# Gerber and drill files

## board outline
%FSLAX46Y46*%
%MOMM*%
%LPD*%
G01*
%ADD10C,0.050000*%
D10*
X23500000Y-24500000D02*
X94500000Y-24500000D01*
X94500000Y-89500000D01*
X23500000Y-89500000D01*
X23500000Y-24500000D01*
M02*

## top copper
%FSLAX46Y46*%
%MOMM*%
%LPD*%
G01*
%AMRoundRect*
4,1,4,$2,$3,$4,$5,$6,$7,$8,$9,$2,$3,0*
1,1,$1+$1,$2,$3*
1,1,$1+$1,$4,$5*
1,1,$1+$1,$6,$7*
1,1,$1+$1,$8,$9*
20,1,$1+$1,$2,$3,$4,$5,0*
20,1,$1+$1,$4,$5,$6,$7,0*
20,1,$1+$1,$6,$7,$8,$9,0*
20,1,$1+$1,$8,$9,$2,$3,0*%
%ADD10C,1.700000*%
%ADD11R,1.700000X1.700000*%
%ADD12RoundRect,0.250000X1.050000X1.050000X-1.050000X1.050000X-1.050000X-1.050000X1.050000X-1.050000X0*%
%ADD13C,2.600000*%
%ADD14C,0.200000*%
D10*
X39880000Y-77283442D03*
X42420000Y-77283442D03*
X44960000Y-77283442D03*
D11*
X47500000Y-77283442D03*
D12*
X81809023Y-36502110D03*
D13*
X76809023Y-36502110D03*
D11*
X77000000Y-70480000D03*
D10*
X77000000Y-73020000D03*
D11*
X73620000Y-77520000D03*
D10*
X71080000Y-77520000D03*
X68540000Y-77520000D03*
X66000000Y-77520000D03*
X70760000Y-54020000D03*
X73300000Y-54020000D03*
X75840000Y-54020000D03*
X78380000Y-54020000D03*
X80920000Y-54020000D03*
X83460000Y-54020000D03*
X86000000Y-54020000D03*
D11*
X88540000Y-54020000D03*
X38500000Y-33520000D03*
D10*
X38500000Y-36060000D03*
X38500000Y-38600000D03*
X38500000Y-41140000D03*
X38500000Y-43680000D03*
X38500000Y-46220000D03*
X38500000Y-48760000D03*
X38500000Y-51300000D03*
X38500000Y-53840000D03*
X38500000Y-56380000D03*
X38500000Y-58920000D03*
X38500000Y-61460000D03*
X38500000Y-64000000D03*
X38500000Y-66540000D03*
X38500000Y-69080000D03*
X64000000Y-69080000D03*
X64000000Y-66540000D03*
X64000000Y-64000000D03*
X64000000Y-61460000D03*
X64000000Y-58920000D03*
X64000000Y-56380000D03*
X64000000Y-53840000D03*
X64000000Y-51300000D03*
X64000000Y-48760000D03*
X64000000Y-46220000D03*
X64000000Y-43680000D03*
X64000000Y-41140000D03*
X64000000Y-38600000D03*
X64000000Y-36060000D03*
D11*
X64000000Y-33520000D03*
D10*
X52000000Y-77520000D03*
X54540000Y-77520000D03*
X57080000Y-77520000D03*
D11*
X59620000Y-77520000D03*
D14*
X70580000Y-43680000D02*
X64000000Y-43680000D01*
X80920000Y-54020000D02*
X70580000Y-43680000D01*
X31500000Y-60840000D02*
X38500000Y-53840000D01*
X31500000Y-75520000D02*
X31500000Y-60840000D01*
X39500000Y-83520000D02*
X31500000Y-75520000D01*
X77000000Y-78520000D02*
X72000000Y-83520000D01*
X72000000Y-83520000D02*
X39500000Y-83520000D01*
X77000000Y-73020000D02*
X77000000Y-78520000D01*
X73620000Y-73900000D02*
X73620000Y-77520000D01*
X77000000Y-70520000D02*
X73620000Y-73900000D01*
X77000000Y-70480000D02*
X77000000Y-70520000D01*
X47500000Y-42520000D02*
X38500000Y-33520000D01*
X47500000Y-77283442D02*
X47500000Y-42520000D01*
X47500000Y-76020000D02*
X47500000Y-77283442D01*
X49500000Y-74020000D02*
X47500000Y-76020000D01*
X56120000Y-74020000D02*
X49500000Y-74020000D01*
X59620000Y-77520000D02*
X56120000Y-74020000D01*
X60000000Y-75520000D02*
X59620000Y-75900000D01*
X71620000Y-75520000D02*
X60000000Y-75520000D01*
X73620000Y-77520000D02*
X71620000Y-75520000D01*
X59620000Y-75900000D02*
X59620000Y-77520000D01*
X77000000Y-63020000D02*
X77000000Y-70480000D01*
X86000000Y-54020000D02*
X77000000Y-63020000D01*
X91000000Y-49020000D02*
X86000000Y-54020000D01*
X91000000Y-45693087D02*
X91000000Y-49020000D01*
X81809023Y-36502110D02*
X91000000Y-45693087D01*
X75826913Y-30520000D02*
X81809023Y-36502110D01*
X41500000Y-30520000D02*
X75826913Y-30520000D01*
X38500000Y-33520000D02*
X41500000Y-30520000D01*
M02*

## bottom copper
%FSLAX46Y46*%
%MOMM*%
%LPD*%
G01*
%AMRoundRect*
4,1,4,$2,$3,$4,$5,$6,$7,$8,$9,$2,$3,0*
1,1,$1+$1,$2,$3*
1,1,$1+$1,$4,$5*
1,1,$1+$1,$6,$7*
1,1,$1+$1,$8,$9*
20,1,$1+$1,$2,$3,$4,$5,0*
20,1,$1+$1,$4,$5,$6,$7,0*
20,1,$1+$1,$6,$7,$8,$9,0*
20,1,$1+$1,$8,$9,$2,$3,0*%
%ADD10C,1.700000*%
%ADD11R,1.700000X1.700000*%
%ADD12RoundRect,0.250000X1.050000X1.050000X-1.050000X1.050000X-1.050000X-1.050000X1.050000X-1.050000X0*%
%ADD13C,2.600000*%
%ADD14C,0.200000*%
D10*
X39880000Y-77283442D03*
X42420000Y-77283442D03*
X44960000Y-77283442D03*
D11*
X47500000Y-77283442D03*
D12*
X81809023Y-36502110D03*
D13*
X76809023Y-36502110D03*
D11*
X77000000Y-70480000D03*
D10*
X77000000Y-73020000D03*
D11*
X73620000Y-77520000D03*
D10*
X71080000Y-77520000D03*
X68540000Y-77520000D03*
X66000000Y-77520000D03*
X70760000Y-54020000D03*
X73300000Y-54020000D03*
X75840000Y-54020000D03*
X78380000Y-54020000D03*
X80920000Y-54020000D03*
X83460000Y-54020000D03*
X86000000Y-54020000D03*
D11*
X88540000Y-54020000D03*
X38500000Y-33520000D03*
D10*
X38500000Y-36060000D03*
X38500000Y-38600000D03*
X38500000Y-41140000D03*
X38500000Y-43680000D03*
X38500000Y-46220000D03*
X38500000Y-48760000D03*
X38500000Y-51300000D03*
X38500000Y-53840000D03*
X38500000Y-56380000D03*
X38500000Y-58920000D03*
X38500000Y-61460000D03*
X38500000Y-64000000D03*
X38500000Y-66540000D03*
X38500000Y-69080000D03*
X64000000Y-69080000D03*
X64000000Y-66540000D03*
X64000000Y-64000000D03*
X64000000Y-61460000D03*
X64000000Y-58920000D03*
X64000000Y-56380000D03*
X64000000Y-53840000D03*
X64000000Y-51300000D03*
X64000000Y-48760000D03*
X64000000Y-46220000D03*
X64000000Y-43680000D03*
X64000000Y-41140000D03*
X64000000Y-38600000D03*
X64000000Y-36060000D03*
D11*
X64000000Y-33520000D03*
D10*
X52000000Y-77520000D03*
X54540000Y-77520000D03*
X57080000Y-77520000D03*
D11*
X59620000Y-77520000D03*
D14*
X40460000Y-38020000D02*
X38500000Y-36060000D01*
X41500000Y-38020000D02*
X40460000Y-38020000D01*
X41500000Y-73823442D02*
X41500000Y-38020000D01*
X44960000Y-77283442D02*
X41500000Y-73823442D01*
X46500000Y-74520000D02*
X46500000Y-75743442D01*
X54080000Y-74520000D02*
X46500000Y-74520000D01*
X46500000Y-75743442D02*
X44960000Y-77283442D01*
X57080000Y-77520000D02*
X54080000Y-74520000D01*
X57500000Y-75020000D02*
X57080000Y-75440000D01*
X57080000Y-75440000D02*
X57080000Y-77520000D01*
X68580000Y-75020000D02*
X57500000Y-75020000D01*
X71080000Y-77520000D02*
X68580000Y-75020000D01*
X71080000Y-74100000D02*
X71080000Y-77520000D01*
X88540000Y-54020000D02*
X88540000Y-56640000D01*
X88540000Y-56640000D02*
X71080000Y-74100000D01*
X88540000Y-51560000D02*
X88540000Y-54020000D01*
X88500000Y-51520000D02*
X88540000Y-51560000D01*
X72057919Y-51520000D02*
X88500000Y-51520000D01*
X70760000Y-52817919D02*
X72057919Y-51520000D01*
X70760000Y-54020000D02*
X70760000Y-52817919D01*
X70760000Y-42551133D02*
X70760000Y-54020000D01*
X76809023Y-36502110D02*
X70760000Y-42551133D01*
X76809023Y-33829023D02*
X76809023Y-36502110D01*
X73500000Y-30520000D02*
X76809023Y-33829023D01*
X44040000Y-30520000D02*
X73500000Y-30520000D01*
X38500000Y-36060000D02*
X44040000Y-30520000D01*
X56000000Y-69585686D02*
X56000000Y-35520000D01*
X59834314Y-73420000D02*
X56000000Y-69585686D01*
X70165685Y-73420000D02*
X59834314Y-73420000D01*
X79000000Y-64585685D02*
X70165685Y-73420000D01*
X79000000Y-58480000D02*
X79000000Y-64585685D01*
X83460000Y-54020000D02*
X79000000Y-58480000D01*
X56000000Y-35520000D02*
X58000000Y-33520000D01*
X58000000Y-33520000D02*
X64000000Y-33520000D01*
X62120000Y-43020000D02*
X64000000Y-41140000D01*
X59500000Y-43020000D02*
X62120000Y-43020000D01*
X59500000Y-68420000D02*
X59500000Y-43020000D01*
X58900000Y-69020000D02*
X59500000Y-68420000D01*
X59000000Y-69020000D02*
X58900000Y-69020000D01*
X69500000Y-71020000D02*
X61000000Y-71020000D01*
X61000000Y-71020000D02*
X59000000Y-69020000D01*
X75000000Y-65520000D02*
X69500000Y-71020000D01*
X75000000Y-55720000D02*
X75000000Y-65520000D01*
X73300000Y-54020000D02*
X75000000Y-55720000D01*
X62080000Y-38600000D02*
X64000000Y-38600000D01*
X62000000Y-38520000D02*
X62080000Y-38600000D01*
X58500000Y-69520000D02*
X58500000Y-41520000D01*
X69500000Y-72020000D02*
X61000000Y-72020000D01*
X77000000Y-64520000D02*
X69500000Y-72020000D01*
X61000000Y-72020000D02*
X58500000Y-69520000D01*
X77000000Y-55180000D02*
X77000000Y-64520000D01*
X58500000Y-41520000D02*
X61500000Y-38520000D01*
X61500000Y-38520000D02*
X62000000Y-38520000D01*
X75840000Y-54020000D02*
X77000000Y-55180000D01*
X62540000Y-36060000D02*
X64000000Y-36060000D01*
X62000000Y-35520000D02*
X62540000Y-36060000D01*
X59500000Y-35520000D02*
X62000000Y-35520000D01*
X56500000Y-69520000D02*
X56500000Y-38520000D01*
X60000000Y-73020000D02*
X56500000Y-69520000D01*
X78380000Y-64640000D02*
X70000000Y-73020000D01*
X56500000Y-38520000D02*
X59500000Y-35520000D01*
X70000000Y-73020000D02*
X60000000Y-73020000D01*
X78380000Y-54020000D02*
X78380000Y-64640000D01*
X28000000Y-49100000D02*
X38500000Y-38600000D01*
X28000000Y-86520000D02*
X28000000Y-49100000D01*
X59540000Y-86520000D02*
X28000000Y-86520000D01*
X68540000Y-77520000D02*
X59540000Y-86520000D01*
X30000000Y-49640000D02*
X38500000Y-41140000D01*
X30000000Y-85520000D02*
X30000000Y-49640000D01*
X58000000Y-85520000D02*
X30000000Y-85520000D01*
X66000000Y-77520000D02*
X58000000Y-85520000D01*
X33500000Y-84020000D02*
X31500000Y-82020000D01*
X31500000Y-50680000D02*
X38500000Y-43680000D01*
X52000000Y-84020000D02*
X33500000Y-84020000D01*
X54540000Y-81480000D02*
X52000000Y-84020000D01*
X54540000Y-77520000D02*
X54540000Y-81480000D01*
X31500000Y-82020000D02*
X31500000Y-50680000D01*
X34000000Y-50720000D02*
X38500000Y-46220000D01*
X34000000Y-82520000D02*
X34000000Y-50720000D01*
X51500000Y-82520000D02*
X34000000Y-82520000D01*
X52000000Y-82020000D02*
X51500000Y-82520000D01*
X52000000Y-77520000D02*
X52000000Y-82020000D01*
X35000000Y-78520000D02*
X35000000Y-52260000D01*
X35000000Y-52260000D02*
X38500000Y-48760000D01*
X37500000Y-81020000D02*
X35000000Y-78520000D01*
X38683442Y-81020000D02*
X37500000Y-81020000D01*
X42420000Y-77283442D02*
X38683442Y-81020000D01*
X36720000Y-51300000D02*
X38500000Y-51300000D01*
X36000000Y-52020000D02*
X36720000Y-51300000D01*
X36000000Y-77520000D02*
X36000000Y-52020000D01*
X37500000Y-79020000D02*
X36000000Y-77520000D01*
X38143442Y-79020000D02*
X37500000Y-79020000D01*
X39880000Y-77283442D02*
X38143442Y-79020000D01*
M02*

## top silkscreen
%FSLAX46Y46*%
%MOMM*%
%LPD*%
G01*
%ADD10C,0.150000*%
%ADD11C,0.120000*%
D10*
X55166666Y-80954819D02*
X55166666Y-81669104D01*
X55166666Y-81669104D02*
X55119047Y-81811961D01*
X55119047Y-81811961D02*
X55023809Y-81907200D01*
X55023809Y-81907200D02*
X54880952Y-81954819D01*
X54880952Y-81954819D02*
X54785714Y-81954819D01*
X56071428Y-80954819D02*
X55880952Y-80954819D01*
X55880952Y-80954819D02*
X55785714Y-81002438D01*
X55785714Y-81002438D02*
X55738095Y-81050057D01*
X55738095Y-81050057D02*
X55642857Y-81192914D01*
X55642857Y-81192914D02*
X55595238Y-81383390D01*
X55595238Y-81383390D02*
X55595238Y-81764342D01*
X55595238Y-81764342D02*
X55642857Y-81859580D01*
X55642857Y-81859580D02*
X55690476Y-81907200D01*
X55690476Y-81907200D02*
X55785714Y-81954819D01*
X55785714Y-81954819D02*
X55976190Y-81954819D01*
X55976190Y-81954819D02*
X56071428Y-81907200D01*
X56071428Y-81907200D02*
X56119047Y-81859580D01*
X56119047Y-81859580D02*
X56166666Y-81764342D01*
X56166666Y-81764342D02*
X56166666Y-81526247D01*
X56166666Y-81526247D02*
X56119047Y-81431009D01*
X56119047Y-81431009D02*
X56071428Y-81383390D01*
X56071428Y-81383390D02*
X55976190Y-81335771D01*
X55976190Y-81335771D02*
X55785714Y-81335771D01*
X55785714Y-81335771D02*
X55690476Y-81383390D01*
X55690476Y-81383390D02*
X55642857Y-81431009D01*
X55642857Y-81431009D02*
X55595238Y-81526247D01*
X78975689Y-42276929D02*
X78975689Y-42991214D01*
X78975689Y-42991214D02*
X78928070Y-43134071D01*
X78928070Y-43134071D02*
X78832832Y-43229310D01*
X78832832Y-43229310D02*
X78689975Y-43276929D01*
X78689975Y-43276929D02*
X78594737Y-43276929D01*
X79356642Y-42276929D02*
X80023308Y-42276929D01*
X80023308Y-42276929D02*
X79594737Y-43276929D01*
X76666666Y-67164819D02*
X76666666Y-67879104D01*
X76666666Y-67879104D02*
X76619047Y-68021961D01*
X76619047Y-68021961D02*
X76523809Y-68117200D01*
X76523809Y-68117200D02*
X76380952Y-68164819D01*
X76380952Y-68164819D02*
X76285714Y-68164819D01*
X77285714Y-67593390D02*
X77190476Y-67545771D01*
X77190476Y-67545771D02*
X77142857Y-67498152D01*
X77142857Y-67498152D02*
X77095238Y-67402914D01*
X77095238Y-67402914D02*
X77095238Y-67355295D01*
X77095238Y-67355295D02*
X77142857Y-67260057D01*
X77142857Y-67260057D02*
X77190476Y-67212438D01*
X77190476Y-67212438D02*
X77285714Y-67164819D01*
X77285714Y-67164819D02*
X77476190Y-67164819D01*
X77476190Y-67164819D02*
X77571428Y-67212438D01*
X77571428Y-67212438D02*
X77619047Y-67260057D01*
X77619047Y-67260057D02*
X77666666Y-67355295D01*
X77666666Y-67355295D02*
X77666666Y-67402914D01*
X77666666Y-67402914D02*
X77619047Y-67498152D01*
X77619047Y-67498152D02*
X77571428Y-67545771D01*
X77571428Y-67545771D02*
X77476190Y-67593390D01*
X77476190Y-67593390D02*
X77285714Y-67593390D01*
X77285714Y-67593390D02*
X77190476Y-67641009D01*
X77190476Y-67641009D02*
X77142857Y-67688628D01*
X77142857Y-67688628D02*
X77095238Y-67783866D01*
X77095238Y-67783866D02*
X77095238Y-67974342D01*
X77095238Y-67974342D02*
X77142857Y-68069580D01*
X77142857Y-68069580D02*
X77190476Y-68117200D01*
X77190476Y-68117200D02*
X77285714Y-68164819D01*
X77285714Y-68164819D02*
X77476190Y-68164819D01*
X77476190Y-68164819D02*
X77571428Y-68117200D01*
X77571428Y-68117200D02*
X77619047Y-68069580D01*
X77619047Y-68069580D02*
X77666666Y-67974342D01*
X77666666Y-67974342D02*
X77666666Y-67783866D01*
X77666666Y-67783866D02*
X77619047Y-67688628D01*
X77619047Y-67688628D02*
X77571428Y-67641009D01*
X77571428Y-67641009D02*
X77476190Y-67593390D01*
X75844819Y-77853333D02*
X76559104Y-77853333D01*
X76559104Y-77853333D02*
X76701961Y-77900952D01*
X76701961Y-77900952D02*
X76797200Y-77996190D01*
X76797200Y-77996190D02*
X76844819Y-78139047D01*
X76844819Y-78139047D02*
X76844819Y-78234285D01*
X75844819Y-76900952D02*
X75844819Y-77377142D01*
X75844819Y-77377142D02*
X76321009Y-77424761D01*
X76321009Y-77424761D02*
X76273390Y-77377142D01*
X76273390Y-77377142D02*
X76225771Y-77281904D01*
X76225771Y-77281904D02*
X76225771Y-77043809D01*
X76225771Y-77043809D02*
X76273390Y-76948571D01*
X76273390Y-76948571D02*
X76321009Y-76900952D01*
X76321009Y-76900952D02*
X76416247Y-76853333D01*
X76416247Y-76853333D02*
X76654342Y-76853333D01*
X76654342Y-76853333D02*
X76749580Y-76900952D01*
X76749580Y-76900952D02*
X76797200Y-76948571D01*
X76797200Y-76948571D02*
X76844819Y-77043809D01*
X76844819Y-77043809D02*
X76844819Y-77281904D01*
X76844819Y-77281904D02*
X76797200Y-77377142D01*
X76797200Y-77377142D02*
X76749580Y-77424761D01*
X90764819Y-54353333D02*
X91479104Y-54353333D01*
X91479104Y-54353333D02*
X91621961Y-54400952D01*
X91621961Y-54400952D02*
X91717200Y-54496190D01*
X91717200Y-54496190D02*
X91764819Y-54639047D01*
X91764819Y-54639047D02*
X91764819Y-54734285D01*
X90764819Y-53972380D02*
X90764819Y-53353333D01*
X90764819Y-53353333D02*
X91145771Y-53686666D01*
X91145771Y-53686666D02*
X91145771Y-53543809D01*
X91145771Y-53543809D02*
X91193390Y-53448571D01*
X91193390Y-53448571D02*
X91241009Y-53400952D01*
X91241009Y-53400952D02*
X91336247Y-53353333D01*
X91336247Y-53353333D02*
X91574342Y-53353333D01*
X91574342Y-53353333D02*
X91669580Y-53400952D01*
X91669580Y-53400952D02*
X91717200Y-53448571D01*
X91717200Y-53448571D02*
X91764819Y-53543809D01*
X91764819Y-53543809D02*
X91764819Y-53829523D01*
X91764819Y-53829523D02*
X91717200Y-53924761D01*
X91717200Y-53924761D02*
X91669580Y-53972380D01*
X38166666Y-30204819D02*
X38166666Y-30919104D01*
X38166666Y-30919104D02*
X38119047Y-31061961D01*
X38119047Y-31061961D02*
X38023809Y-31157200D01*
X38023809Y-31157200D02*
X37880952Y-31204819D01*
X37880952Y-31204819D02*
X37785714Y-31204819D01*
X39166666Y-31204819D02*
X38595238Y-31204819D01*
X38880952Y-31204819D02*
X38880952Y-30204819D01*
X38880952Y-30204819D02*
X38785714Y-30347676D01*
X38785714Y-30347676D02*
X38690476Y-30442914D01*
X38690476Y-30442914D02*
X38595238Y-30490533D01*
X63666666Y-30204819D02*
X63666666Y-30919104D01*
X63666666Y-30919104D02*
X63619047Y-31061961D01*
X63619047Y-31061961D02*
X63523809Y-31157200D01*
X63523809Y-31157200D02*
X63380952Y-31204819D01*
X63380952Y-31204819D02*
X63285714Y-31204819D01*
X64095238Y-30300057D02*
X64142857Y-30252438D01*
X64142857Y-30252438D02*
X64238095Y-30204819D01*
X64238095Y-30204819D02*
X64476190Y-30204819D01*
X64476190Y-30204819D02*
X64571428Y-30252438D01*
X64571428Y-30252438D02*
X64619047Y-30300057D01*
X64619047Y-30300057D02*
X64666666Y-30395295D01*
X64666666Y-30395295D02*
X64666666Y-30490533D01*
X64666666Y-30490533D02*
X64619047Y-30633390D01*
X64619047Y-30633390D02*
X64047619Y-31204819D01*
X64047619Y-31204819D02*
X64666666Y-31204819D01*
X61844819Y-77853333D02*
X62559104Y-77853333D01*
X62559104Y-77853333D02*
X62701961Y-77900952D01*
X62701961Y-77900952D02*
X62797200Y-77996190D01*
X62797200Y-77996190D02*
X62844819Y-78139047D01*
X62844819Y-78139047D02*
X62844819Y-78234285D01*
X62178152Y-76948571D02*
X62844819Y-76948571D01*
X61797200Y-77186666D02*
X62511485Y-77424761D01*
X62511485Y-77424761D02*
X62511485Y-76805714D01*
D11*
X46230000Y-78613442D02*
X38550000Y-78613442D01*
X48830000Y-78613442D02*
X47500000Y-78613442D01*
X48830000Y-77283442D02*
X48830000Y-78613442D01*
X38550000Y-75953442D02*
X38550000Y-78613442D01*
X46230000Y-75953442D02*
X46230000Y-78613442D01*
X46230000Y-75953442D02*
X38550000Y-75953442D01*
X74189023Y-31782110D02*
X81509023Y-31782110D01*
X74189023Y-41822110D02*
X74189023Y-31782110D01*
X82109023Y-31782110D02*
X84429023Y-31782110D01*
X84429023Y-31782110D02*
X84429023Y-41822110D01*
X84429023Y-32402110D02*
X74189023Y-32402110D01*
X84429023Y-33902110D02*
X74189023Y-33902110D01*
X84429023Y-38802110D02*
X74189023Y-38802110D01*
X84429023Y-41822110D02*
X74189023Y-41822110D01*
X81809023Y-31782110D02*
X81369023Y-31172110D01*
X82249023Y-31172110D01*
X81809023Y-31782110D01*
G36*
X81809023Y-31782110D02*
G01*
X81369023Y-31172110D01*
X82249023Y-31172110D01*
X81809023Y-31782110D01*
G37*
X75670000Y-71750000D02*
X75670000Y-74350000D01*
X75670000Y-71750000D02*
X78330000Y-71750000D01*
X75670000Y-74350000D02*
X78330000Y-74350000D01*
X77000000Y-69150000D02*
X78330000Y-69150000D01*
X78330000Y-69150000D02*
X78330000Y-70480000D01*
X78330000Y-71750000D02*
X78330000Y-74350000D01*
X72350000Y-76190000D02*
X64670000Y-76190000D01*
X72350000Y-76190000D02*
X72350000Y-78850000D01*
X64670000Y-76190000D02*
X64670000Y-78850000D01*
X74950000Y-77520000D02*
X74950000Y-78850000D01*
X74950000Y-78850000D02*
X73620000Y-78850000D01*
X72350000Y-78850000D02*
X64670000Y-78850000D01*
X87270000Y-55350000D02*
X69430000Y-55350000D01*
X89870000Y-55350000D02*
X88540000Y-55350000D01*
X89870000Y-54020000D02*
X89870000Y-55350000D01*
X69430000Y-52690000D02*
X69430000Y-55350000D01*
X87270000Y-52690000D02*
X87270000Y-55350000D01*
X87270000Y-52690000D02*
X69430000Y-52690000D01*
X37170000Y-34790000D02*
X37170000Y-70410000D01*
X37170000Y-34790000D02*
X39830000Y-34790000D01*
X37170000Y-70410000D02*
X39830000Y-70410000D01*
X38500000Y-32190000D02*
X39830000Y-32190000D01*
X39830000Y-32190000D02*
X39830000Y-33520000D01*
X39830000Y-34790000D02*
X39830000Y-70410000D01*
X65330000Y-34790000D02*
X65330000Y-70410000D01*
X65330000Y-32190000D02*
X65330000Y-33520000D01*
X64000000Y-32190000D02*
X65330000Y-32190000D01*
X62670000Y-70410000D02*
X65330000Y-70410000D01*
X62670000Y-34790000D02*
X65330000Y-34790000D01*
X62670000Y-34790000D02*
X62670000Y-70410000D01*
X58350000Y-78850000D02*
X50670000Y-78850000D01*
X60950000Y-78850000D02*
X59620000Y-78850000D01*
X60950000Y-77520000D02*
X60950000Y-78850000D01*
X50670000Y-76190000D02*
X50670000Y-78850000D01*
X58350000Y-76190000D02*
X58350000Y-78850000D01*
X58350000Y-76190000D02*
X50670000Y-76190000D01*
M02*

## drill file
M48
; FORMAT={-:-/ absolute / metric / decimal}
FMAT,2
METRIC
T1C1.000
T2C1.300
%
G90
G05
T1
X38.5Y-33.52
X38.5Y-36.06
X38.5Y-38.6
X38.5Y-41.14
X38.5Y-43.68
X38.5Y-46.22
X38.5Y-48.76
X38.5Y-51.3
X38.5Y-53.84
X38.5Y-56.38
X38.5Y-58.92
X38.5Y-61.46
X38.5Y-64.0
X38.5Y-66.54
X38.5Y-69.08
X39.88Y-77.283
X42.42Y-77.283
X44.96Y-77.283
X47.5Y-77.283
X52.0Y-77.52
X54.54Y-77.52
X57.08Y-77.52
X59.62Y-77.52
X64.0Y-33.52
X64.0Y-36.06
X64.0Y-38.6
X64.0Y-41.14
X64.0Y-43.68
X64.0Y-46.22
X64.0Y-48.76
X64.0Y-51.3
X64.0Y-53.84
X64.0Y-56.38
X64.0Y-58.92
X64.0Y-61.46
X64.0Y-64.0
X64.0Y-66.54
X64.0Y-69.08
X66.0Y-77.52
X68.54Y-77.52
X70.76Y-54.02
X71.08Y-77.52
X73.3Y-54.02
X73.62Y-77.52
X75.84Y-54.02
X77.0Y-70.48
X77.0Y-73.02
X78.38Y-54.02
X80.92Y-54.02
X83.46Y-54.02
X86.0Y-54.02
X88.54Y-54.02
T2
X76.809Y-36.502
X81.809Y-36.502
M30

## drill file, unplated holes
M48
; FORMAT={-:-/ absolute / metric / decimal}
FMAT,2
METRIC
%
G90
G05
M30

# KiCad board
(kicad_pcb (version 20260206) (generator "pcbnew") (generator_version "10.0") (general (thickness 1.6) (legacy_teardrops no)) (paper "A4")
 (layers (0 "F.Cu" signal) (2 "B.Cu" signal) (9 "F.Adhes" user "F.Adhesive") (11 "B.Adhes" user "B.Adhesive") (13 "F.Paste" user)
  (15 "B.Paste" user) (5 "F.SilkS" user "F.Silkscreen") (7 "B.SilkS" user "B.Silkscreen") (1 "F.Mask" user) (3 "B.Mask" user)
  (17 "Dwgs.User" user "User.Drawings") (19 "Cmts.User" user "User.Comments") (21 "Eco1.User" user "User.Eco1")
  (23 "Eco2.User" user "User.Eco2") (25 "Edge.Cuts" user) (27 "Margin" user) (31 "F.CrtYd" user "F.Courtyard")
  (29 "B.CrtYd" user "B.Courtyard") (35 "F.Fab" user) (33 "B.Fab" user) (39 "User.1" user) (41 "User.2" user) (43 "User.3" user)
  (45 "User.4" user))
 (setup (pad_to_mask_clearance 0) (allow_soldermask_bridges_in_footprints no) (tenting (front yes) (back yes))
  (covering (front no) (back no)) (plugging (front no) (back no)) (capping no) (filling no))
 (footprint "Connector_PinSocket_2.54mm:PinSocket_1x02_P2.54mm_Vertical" (layer "F.Cu") (at 77 70.48)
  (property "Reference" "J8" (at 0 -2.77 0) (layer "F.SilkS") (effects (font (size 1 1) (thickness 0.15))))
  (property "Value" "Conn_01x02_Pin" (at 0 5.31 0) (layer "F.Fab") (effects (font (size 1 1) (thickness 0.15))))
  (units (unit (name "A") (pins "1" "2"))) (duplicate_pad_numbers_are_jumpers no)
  (fp_line (start -1.33 1.27) (end -1.33 3.87) (stroke (width 0.12) (type solid)) (layer "F.SilkS"))
  (fp_line (start -1.33 1.27) (end 1.33 1.27) (stroke (width 0.12) (type solid)) (layer "F.SilkS"))
  (fp_line (start -1.33 3.87) (end 1.33 3.87) (stroke (width 0.12) (type solid)) (layer "F.SilkS"))
  (fp_line (start 0 -1.33) (end 1.33 -1.33) (stroke (width 0.12) (type solid)) (layer "F.SilkS"))
  (fp_line (start 1.33 -1.33) (end 1.33 0) (stroke (width 0.12) (type solid)) (layer "F.SilkS"))
  (fp_line (start 1.33 1.27) (end 1.33 3.87) (stroke (width 0.12) (type solid)) (layer "F.SilkS"))
  (pad "1" thru_hole rect (at 0 0) (size 1.7 1.7) (drill 1) (layers "*.Cu" "*.Mask") (remove_unused_layers no) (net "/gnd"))
  (pad "2" thru_hole circle (at 0 2.54) (size 1.7 1.7) (drill 1) (layers "*.Cu" "*.Mask") (remove_unused_layers no) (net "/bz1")))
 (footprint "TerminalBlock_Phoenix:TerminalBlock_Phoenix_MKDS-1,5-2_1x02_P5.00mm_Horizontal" (layer "F.Cu") (at 81.809023 36.50211 180)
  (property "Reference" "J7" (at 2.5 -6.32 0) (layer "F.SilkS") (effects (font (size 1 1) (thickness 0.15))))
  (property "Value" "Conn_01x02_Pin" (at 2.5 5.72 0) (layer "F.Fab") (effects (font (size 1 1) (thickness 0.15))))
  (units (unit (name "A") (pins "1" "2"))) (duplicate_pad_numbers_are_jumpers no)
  (fp_line (start 7.62 4.72) (end 0.3 4.72) (stroke (width 0.12) (type solid)) (layer "F.SilkS"))
  (fp_line (start 7.62 -5.32) (end 7.62 4.72) (stroke (width 0.12) (type solid)) (layer "F.SilkS"))
  (fp_line (start -0.3 4.72) (end -2.62 4.72) (stroke (width 0.12) (type solid)) (layer "F.SilkS"))
  (fp_line (start -2.62 4.72) (end -2.62 -5.32) (stroke (width 0.12) (type solid)) (layer "F.SilkS"))
  (fp_line (start -2.62 4.1) (end 7.62 4.1) (stroke (width 0.12) (type solid)) (layer "F.SilkS"))
  (fp_line (start -2.62 2.6) (end 7.62 2.6) (stroke (width 0.12) (type solid)) (layer "F.SilkS"))
  (fp_line (start -2.62 -2.3) (end 7.62 -2.3) (stroke (width 0.12) (type solid)) (layer "F.SilkS"))
  (fp_line (start -2.62 -5.32) (end 7.62 -5.32) (stroke (width 0.12) (type solid)) (layer "F.SilkS"))
  (fp_poly (pts (xy 0 4.72) (xy 0.44 5.33) (xy -0.44 5.33)) (stroke (width 0.12) (type solid)) (fill yes) (layer "F.SilkS"))
  (pad "1" thru_hole roundrect (at 0 0 180) (size 2.6 2.6) (drill 1.3) (layers "*.Cu" "*.Mask") (remove_unused_layers no)
   (roundrect_rratio 0.096154) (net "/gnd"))
  (pad "2" thru_hole circle (at 5 0 180) (size 2.6 2.6) (drill 1.3) (layers "*.Cu" "*.Mask") (remove_unused_layers no) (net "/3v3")))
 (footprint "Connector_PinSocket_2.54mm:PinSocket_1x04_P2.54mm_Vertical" (layer "F.Cu") (at 73.62 77.52 -90)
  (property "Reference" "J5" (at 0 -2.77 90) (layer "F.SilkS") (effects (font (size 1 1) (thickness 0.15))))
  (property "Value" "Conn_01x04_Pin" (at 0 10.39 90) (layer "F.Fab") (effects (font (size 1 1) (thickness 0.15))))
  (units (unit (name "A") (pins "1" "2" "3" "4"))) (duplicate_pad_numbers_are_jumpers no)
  (fp_line (start -1.33 8.95) (end 1.33 8.95) (stroke (width 0.12) (type solid)) (layer "F.SilkS"))
  (fp_line (start -1.33 1.27) (end -1.33 8.95) (stroke (width 0.12) (type solid)) (layer "F.SilkS"))
  (fp_line (start -1.33 1.27) (end 1.33 1.27) (stroke (width 0.12) (type solid)) (layer "F.SilkS"))
  (fp_line (start 1.33 1.27) (end 1.33 8.95) (stroke (width 0.12) (type solid)) (layer "F.SilkS"))
  (fp_line (start 0 -1.33) (end 1.33 -1.33) (stroke (width 0.12) (type solid)) (layer "F.SilkS"))
  (fp_line (start 1.33 -1.33) (end 1.33 0) (stroke (width 0.12) (type solid)) (layer "F.SilkS"))
  (pad "1" thru_hole rect (at 0 0 270) (size 1.7 1.7) (drill 1) (layers "*.Cu" "*.Mask") (remove_unused_layers no) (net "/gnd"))
  (pad "2" thru_hole circle (at 0 2.54 270) (size 1.7 1.7) (drill 1) (layers "*.Cu" "*.Mask") (remove_unused_layers no) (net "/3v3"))
  (pad "3" thru_hole circle (at 0 5.08 270) (size 1.7 1.7) (drill 1) (layers "*.Cu" "*.Mask") (remove_unused_layers no) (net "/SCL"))
  (pad "4" thru_hole circle (at 0 7.62 270) (size 1.7 1.7) (drill 1) (layers "*.Cu" "*.Mask") (remove_unused_layers no) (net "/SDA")))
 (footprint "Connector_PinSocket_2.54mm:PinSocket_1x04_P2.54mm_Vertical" (layer "F.Cu") (at 47.5 77.283442 -90)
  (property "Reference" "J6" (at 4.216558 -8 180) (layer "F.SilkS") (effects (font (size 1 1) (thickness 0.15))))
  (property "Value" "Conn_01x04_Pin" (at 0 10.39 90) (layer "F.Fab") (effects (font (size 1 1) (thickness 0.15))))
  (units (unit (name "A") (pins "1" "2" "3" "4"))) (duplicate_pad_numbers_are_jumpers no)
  (fp_line (start -1.33 8.95) (end 1.33 8.95) (stroke (width 0.12) (type solid)) (layer "F.SilkS"))
  (fp_line (start -1.33 1.27) (end -1.33 8.95) (stroke (width 0.12) (type solid)) (layer "F.SilkS"))
  (fp_line (start -1.33 1.27) (end 1.33 1.27) (stroke (width 0.12) (type solid)) (layer "F.SilkS"))
  (fp_line (start 1.33 1.27) (end 1.33 8.95) (stroke (width 0.12) (type solid)) (layer "F.SilkS"))
  (fp_line (start 0 -1.33) (end 1.33 -1.33) (stroke (width 0.12) (type solid)) (layer "F.SilkS"))
  (fp_line (start 1.33 -1.33) (end 1.33 0) (stroke (width 0.12) (type solid)) (layer "F.SilkS"))
  (pad "1" thru_hole rect (at 0 0 270) (size 1.7 1.7) (drill 1) (layers "*.Cu" "*.Mask") (remove_unused_layers no) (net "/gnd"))
  (pad "2" thru_hole circle (at 0 2.54 270) (size 1.7 1.7) (drill 1) (layers "*.Cu" "*.Mask") (remove_unused_layers no) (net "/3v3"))
  (pad "3" thru_hole circle (at 0 5.08 270) (size 1.7 1.7) (drill 1) (layers "*.Cu" "*.Mask") (remove_unused_layers no) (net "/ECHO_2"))
  (pad "4" thru_hole circle (at 0 7.62 270) (size 1.7 1.7) (drill 1) (layers "*.Cu" "*.Mask") (remove_unused_layers no) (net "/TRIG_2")))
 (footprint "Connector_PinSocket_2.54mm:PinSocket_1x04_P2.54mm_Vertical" (layer "F.Cu") (at 59.62 77.52 -90)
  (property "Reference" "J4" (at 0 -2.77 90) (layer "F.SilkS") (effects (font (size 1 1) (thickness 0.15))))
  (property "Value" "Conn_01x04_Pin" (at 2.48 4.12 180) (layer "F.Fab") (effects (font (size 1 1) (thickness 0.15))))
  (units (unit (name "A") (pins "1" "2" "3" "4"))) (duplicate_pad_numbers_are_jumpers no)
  (fp_line (start -1.33 8.95) (end 1.33 8.95) (stroke (width 0.12) (type solid)) (layer "F.SilkS"))
  (fp_line (start -1.33 1.27) (end -1.33 8.95) (stroke (width 0.12) (type solid)) (layer "F.SilkS"))
  (fp_line (start -1.33 1.27) (end 1.33 1.27) (stroke (width 0.12) (type solid)) (layer "F.SilkS"))
  (fp_line (start 1.33 1.27) (end 1.33 8.95) (stroke (width 0.12) (type solid)) (layer "F.SilkS"))
  (fp_line (start 0 -1.33) (end 1.33 -1.33) (stroke (width 0.12) (type solid)) (layer "F.SilkS"))
  (fp_line (start 1.33 -1.33) (end 1.33 0) (stroke (width 0.12) (type solid)) (layer "F.SilkS"))
  (pad "1" thru_hole rect (at 0 0 270) (size 1.7 1.7) (drill 1) (layers "*.Cu" "*.Mask") (remove_unused_layers no) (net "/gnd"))
  (pad "2" thru_hole circle (at 0 2.54 270) (size 1.7 1.7) (drill 1) (layers "*.Cu" "*.Mask") (remove_unused_layers no) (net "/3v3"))
  (pad "3" thru_hole circle (at 0 5.08 270) (size 1.7 1.7) (drill 1) (layers "*.Cu" "*.Mask") (remove_unused_layers no) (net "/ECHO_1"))
  (pad "4" thru_hole circle (at 0 7.62 270) (size 1.7 1.7) (drill 1) (layers "*.Cu" "*.Mask") (remove_unused_layers no) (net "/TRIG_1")))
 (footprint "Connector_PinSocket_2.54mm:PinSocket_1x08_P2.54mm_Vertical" (layer "F.Cu") (at 88.54 54.02 -90)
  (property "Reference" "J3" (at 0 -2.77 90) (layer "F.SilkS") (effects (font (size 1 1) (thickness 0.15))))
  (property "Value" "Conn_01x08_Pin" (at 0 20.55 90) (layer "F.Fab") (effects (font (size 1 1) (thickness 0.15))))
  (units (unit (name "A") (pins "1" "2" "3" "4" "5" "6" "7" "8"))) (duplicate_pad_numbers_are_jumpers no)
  (fp_line (start -1.33 19.11) (end 1.33 19.11) (stroke (width 0.12) (type solid)) (layer "F.SilkS"))
  (fp_line (start -1.33 1.27) (end -1.33 19.11) (stroke (width 0.12) (type solid)) (layer "F.SilkS"))
  (fp_line (start -1.33 1.27) (end 1.33 1.27) (stroke (width 0.12) (type solid)) (layer "F.SilkS"))
  (fp_line (start 1.33 1.27) (end 1.33 19.11) (stroke (width 0.12) (type solid)) (layer "F.SilkS"))
  (fp_line (start 0 -1.33) (end 1.33 -1.33) (stroke (width 0.12) (type solid)) (layer "F.SilkS"))
  (fp_line (start 1.33 -1.33) (end 1.33 0) (stroke (width 0.12) (type solid)) (layer "F.SilkS"))
  (pad "1" thru_hole rect (at 0 0 270) (size 1.7 1.7) (drill 1) (layers "*.Cu" "*.Mask") (remove_unused_layers no) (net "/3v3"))
  (pad "2" thru_hole circle (at 0 2.54 270) (size 1.7 1.7) (drill 1) (layers "*.Cu" "*.Mask") (remove_unused_layers no) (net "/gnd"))
  (pad "3" thru_hole circle (at 0 5.08 270) (size 1.7 1.7) (drill 1) (layers "*.Cu" "*.Mask") (remove_unused_layers no) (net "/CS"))
  (pad "4" thru_hole circle (at 0 7.62 270) (size 1.7 1.7) (drill 1) (layers "*.Cu" "*.Mask") (remove_unused_layers no) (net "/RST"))
  (pad "5" thru_hole circle (at 0 10.16 270) (size 1.7 1.7) (drill 1) (layers "*.Cu" "*.Mask") (remove_unused_layers no) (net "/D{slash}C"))
  (pad "6" thru_hole circle (at 0 12.7 270) (size 1.7 1.7) (drill 1) (layers "*.Cu" "*.Mask") (remove_unused_layers no) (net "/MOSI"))
  (pad "7" thru_hole circle (at 0 15.24 270) (size 1.7 1.7) (drill 1) (layers "*.Cu" "*.Mask") (remove_unused_layers no) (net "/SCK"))
  (pad "8" thru_hole circle (at 0 17.78 270) (size 1.7 1.7) (drill 1) (layers "*.Cu" "*.Mask") (remove_unused_layers no) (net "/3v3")))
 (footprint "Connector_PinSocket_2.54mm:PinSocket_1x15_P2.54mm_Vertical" (layer "F.Cu") (at 38.5 33.52)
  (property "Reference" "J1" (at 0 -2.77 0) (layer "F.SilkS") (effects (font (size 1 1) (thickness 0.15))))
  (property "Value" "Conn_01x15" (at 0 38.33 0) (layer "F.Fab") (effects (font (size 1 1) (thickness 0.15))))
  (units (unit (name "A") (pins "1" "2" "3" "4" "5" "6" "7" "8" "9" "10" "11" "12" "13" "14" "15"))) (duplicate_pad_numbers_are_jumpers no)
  (fp_line (start -1.33 1.27) (end -1.33 36.89) (stroke (width 0.12) (type solid)) (layer "F.SilkS"))
  (fp_line (start -1.33 1.27) (end 1.33 1.27) (stroke (width 0.12) (type solid)) (layer "F.SilkS"))
  (fp_line (start -1.33 36.89) (end 1.33 36.89) (stroke (width 0.12) (type solid)) (layer "F.SilkS"))
  (fp_line (start 0 -1.33) (end 1.33 -1.33) (stroke (width 0.12) (type solid)) (layer "F.SilkS"))
  (fp_line (start 1.33 -1.33) (end 1.33 0) (stroke (width 0.12) (type solid)) (layer "F.SilkS"))
  (fp_line (start 1.33 1.27) (end 1.33 36.89) (stroke (width 0.12) (type solid)) (layer "F.SilkS"))
  (pad "1" thru_hole rect (at 0 0) (size 1.7 1.7) (drill 1) (layers "*.Cu" "*.Mask") (remove_unused_layers no) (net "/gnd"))
  (pad "2" thru_hole circle (at 0 2.54) (size 1.7 1.7) (drill 1) (layers "*.Cu" "*.Mask") (remove_unused_layers no) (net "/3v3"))
  (pad "3" thru_hole circle (at 0 5.08) (size 1.7 1.7) (drill 1) (layers "*.Cu" "*.Mask") (remove_unused_layers no) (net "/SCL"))
  (pad "4" thru_hole circle (at 0 7.62) (size 1.7 1.7) (drill 1) (layers "*.Cu" "*.Mask") (remove_unused_layers no) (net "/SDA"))
  (pad "5" thru_hole circle (at 0 10.16) (size 1.7 1.7) (drill 1) (layers "*.Cu" "*.Mask") (remove_unused_layers no) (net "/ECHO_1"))
  (pad "6" thru_hole circle (at 0 12.7) (size 1.7 1.7) (drill 1) (layers "*.Cu" "*.Mask") (remove_unused_layers no) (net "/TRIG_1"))
  (pad "7" thru_hole circle (at 0 15.24) (size 1.7 1.7) (drill 1) (layers "*.Cu" "*.Mask") (remove_unused_layers no) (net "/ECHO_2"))
  (pad "8" thru_hole circle (at 0 17.78) (size 1.7 1.7) (drill 1) (layers "*.Cu" "*.Mask") (remove_unused_layers no) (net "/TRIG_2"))
  (pad "9" thru_hole circle (at 0 20.32) (size 1.7 1.7) (drill 1) (layers "*.Cu" "*.Mask") (remove_unused_layers no) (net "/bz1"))
  (pad "10" thru_hole circle (at 0 22.86) (size 1.7 1.7) (drill 1) (layers "*.Cu" "*.Mask") (remove_unused_layers no)
   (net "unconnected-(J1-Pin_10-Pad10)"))
  (pad "11" thru_hole circle (at 0 25.4) (size 1.7 1.7) (drill 1) (layers "*.Cu" "*.Mask") (remove_unused_layers no)
   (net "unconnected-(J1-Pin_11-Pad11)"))
  (pad "12" thru_hole circle (at 0 27.94) (size 1.7 1.7) (drill 1) (layers "*.Cu" "*.Mask") (remove_unused_layers no)
   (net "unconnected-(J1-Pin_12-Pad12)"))
  (pad "13" thru_hole circle (at 0 30.48) (size 1.7 1.7) (drill 1) (layers "*.Cu" "*.Mask") (remove_unused_layers no)
   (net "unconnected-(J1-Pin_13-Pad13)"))
  (pad "14" thru_hole circle (at 0 33.02) (size 1.7 1.7) (drill 1) (layers "*.Cu" "*.Mask") (remove_unused_layers no)
   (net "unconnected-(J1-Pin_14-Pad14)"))
  (pad "15" thru_hole circle (at 0 35.56) (size 1.7 1.7) (drill 1) (layers "*.Cu" "*.Mask") (remove_unused_layers no)
   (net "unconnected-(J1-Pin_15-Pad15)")))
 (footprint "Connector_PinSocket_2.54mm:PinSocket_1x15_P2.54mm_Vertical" (layer "F.Cu") (at 64 33.52)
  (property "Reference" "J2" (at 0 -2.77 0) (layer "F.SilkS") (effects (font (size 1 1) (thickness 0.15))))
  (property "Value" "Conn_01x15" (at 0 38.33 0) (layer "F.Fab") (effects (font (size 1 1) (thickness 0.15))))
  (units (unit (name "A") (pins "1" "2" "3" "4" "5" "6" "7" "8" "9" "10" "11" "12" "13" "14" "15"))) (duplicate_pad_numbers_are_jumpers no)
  (fp_line (start -1.33 1.27) (end -1.33 36.89) (stroke (width 0.12) (type solid)) (layer "F.SilkS"))
  (fp_line (start -1.33 1.27) (end 1.33 1.27) (stroke (width 0.12) (type solid)) (layer "F.SilkS"))
  (fp_line (start -1.33 36.89) (end 1.33 36.89) (stroke (width 0.12) (type solid)) (layer "F.SilkS"))
  (fp_line (start 0 -1.33) (end 1.33 -1.33) (stroke (width 0.12) (type solid)) (layer "F.SilkS"))
  (fp_line (start 1.33 -1.33) (end 1.33 0) (stroke (width 0.12) (type solid)) (layer "F.SilkS"))
  (fp_line (start 1.33 1.27) (end 1.33 36.89) (stroke (width 0.12) (type solid)) (layer "F.SilkS"))
  (pad "1" thru_hole rect (at 0 0) (size 1.7 1.7) (drill 1) (layers "*.Cu" "*.Mask") (remove_unused_layers no) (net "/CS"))
  (pad "2" thru_hole circle (at 0 2.54) (size 1.7 1.7) (drill 1) (layers "*.Cu" "*.Mask") (remove_unused_layers no) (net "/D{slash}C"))
  (pad "3" thru_hole circle (at 0 5.08) (size 1.7 1.7) (drill 1) (layers "*.Cu" "*.Mask") (remove_unused_layers no) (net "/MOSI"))
  (pad "4" thru_hole circle (at 0 7.62) (size 1.7 1.7) (drill 1) (layers "*.Cu" "*.Mask") (remove_unused_layers no) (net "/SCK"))
  (pad "5" thru_hole circle (at 0 10.16) (size 1.7 1.7) (drill 1) (layers "*.Cu" "*.Mask") (remove_unused_layers no) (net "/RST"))
  (pad "6" thru_hole circle (at 0 12.7) (size 1.7 1.7) (drill 1) (layers "*.Cu" "*.Mask") (remove_unused_layers no)
   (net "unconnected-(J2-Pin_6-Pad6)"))
  (pad "7" thru_hole circle (at 0 15.24) (size 1.7 1.7) (drill 1) (layers "*.Cu" "*.Mask") (remove_unused_layers no)
   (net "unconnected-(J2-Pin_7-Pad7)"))
  (pad "8" thru_hole circle (at 0 17.78) (size 1.7 1.7) (drill 1) (layers "*.Cu" "*.Mask") (remove_unused_layers no)
   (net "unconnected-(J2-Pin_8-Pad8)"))
  (pad "9" thru_hole circle (at 0 20.32) (size 1.7 1.7) (drill 1) (layers "*.Cu" "*.Mask") (remove_unused_layers no)
   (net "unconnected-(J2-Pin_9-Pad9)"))
  (pad "10" thru_hole circle (at 0 22.86) (size 1.7 1.7) (drill 1) (layers "*.Cu" "*.Mask") (remove_unused_layers no)
   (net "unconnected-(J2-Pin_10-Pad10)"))
  (pad "11" thru_hole circle (at 0 25.4) (size 1.7 1.7) (drill 1) (layers "*.Cu" "*.Mask") (remove_unused_layers no)
   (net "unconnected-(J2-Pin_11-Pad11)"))
  (pad "12" thru_hole circle (at 0 27.94) (size 1.7 1.7) (drill 1) (layers "*.Cu" "*.Mask") (remove_unused_layers no)
   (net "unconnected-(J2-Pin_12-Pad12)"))
  (pad "13" thru_hole circle (at 0 30.48) (size 1.7 1.7) (drill 1) (layers "*.Cu" "*.Mask") (remove_unused_layers no)
   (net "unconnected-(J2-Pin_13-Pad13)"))
  (pad "14" thru_hole circle (at 0 33.02) (size 1.7 1.7) (drill 1) (layers "*.Cu" "*.Mask") (remove_unused_layers no)
   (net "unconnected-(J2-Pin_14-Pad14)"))
  (pad "15" thru_hole circle (at 0 35.56) (size 1.7 1.7) (drill 1) (layers "*.Cu" "*.Mask") (remove_unused_layers no)
   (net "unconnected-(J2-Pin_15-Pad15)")))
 (gr_rect (start 23.5 24.5) (end 94.5 89.5) (stroke (width 0.05) (type default)) (fill no) (layer "Edge.Cuts"))
 (segment (start 91 49.02) (end 86 54.02) (width 0.2) (layer "F.Cu") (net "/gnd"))
 (segment (start 77 70.52) (end 73.62 73.9) (width 0.2) (layer "F.Cu") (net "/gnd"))
 (segment (start 77 70.48) (end 77 70.52) (width 0.2) (layer "F.Cu") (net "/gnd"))
 (segment (start 60 75.52) (end 59.62 75.9) (width 0.2) (layer "F.Cu") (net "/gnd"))
 (segment (start 86 54.02) (end 77 63.02) (width 0.2) (layer "F.Cu") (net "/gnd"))
 (segment (start 47.5 42.52) (end 38.5 33.52) (width 0.2) (layer "F.Cu") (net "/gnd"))
 (segment (start 49.5 74.02) (end 47.5 76.02) (width 0.2) (layer "F.Cu") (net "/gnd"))
 (segment (start 75.826913 30.52) (end 81.809023 36.50211) (width 0.2) (layer "F.Cu") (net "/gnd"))
 (segment (start 91 45.693087) (end 91 49.02) (width 0.2) (layer "F.Cu") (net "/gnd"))
 (segment (start 47.5 76.02) (end 47.5 77.283442) (width 0.2) (layer "F.Cu") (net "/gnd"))
 (segment (start 59.62 77.52) (end 56.12 74.02) (width 0.2) (layer "F.Cu") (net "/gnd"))
 (segment (start 56.12 74.02) (end 49.5 74.02) (width 0.2) (layer "F.Cu") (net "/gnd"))
 (segment (start 81.809023 36.50211) (end 91 45.693087) (width 0.2) (layer "F.Cu") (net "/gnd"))
 (segment (start 41.5 30.52) (end 75.826913 30.52) (width 0.2) (layer "F.Cu") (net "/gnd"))
 (segment (start 73.62 73.9) (end 73.62 77.52) (width 0.2) (layer "F.Cu") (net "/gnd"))
 (segment (start 38.5 33.52) (end 41.5 30.52) (width 0.2) (layer "F.Cu") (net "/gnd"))
 (segment (start 47.5 77.283442) (end 47.5 42.52) (width 0.2) (layer "F.Cu") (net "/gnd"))
 (segment (start 59.62 75.9) (end 59.62 77.52) (width 0.2) (layer "F.Cu") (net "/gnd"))
 (segment (start 71.62 75.52) (end 60 75.52) (width 0.2) (layer "F.Cu") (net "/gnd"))
 (segment (start 77 63.02) (end 77 70.48) (width 0.2) (layer "F.Cu") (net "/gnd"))
 (segment (start 73.62 77.52) (end 71.62 75.52) (width 0.2) (layer "F.Cu") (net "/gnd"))
 (segment (start 77 73.02) (end 77 78.52) (width 0.2) (layer "F.Cu") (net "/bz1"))
 (segment (start 31.5 60.84) (end 38.5 53.84) (width 0.2) (layer "F.Cu") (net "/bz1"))
 (segment (start 39.5 83.52) (end 31.5 75.52) (width 0.2) (layer "F.Cu") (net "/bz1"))
 (segment (start 77 78.52) (end 72 83.52) (width 0.2) (layer "F.Cu") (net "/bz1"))
 (segment (start 72 83.52) (end 39.5 83.52) (width 0.2) (layer "F.Cu") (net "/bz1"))
 (segment (start 31.5 75.52) (end 31.5 60.84) (width 0.2) (layer "F.Cu") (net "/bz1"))
 (segment (start 70.76 42.551133) (end 70.76 54.02) (width 0.2) (layer "B.Cu") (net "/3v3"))
 (segment (start 88.54 51.56) (end 88.54 54.02) (width 0.2) (layer "B.Cu") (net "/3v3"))
 (segment (start 54.08 74.52) (end 46.5 74.52) (width 0.2) (layer "B.Cu") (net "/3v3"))
 (segment (start 71.08 77.52) (end 68.58 75.02) (width 0.2) (layer "B.Cu") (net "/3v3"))
 (segment (start 88.54 56.64) (end 71.08 74.1) (width 0.2) (layer "B.Cu") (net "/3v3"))
 (segment (start 40.46 38.02) (end 38.5 36.06) (width 0.2) (layer "B.Cu") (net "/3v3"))
 (segment (start 68.58 75.02) (end 57.5 75.02) (width 0.2) (layer "B.Cu") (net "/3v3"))
 (segment (start 57.08 77.52) (end 54.08 74.52) (width 0.2) (layer "B.Cu") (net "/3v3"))
 (segment (start 70.76 54.02) (end 70.76 52.817919) (width 0.2) (layer "B.Cu") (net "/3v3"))
 (segment (start 44.96 77.283442) (end 41.5 73.823442) (width 0.2) (layer "B.Cu") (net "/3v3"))
 (segment (start 88.54 54.02) (end 88.54 56.64) (width 0.2) (layer "B.Cu") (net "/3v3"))
 (segment (start 41.5 73.823442) (end 41.5 38.02) (width 0.2) (layer "B.Cu") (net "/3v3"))
 (segment (start 46.5 74.52) (end 46.5 75.743442) (width 0.2) (layer "B.Cu") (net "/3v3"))
 (segment (start 57.08 75.44) (end 57.08 77.52) (width 0.2) (layer "B.Cu") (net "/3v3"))
 (segment (start 76.809023 33.829023) (end 76.809023 36.50211) (width 0.2) (layer "B.Cu") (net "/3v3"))
 (segment (start 41.5 38.02) (end 40.46 38.02) (width 0.2) (layer "B.Cu") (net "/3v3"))
 (segment (start 73.5 30.52) (end 76.809023 33.829023) (width 0.2) (layer "B.Cu") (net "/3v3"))
 (segment (start 76.809023 36.50211) (end 70.76 42.551133) (width 0.2) (layer "B.Cu") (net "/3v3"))
 (segment (start 71.08 74.1) (end 71.08 77.52) (width 0.2) (layer "B.Cu") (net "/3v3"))
 (segment (start 38.5 36.06) (end 44.04 30.52) (width 0.2) (layer "B.Cu") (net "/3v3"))
 (segment (start 70.76 52.817919) (end 72.057919 51.52) (width 0.2) (layer "B.Cu") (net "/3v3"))
 (segment (start 72.057919 51.52) (end 88.5 51.52) (width 0.2) (layer "B.Cu") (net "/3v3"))
 (segment (start 44.04 30.52) (end 73.5 30.52) (width 0.2) (layer "B.Cu") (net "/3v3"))
 (segment (start 46.5 75.743442) (end 44.96 77.283442) (width 0.2) (layer "B.Cu") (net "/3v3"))
 (segment (start 88.5 51.52) (end 88.54 51.56) (width 0.2) (layer "B.Cu") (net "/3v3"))
 (segment (start 57.5 75.02) (end 57.08 75.44) (width 0.2) (layer "B.Cu") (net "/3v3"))
 (segment (start 28 49.1) (end 38.5 38.6) (width 0.2) (layer "B.Cu") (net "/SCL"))
 (segment (start 59.54 86.52) (end 28 86.52) (width 0.2) (layer "B.Cu") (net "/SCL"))
 (segment (start 28 86.52) (end 28 49.1) (width 0.2) (layer "B.Cu") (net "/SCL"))
 (segment (start 68.54 77.52) (end 59.54 86.52) (width 0.2) (layer "B.Cu") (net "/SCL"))
 (segment (start 66 77.52) (end 58 85.52) (width 0.2) (layer "B.Cu") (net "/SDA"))
 (segment (start 58 85.52) (end 30 85.52) (width 0.2) (layer "B.Cu") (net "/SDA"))
 (segment (start 30 85.52) (end 30 49.64) (width 0.2) (layer "B.Cu") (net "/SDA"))
 (segment (start 30 49.64) (end 38.5 41.14) (width 0.2) (layer "B.Cu") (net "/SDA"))
 (segment (start 37.5 81.02) (end 35 78.52) (width 0.2) (layer "B.Cu") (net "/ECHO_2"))
 (segment (start 38.683442 81.02) (end 37.5 81.02) (width 0.2) (layer "B.Cu") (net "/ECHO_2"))
 (segment (start 42.42 77.283442) (end 38.683442 81.02) (width 0.2) (layer "B.Cu") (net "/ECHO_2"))
 (segment (start 35 52.26) (end 38.5 48.76) (width 0.2) (layer "B.Cu") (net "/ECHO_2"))
 (segment (start 35 78.52) (end 35 52.26) (width 0.2) (layer "B.Cu") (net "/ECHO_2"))
 (segment (start 37.5 79.02) (end 36 77.52) (width 0.2) (layer "B.Cu") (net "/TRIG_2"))
 (segment (start 38.143442 79.02) (end 37.5 79.02) (width 0.2) (layer "B.Cu") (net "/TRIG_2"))
 (segment (start 39.88 77.283442) (end 38.143442 79.02) (width 0.2) (layer "B.Cu") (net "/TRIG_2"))
 (segment (start 36 52.02) (end 36.72 51.3) (width 0.2) (layer "B.Cu") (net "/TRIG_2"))
 (segment (start 36 77.52) (end 36 52.02) (width 0.2) (layer "B.Cu") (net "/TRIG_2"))
 (segment (start 36.72 51.3) (end 38.5 51.3) (width 0.2) (layer "B.Cu") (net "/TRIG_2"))
 (segment (start 33.5 84.02) (end 31.5 82.02) (width 0.2) (layer "B.Cu") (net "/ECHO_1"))
 (segment (start 31.5 82.02) (end 31.5 50.68) (width 0.2) (layer "B.Cu") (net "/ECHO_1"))
 (segment (start 31.5 50.68) (end 38.5 43.68) (width 0.2) (layer "B.Cu") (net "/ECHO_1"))
 (segment (start 52 84.02) (end 33.5 84.02) (width 0.2) (layer "B.Cu") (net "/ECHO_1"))
 (segment (start 54.54 77.52) (end 54.54 81.48) (width 0.2) (layer "B.Cu") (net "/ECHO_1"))
 (segment (start 54.54 81.48) (end 52 84.02) (width 0.2) (layer "B.Cu") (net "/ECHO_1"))
 (segment (start 51.5 82.52) (end 34 82.52) (width 0.2) (layer "B.Cu") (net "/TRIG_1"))
 (segment (start 34 50.72) (end 38.5 46.22) (width 0.2) (layer "B.Cu") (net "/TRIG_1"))
 (segment (start 34 82.52) (end 34 50.72) (width 0.2) (layer "B.Cu") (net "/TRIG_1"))
 (segment (start 52 77.52) (end 52 82.02) (width 0.2) (layer "B.Cu") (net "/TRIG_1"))
 (segment (start 52 82.02) (end 51.5 82.52) (width 0.2) (layer "B.Cu") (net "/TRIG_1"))
 (segment (start 70.165685 73.42) (end 59.834314 73.42) (width 0.2) (layer "B.Cu") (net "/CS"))
 (segment (start 58 33.52) (end 64 33.52) (width 0.2) (layer "B.Cu") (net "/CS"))
 (segment (start 83.46 54.02) (end 79 58.48) (width 0.2) (layer "B.Cu") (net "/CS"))
 (segment (start 59.834314 73.42) (end 56 69.585686) (width 0.2) (layer "B.Cu") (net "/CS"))
 (segment (start 56 69.585686) (end 56 35.52) (width 0.2) (layer "B.Cu") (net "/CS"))
 (segment (start 79 58.48) (end 79 64.585685) (width 0.2) (layer "B.Cu") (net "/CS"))
 (segment (start 79 64.585685) (end 70.165685 73.42) (width 0.2) (layer "B.Cu") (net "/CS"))
 (segment (start 56 35.52) (end 58 33.52) (width 0.2) (layer "B.Cu") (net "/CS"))
 (segment (start 70.58 43.68) (end 64 43.68) (width 0.2) (layer "F.Cu") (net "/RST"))
 (segment (start 80.92 54.02) (end 70.58 43.68) (width 0.2) (layer "F.Cu") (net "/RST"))
 (segment (start 62.54 36.06) (end 64 36.06) (width 0.2) (layer "B.Cu") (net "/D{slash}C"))
 (segment (start 56.5 38.52) (end 59.5 35.52) (width 0.2) (layer "B.Cu") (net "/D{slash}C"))
 (segment (start 56.5 69.52) (end 56.5 38.52) (width 0.2) (layer "B.Cu") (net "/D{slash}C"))
 (segment (start 62 35.52) (end 62.54 36.06) (width 0.2) (layer "B.Cu") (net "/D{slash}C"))
 (segment (start 59.5 35.52) (end 62 35.52) (width 0.2) (layer "B.Cu") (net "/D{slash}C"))
 (segment (start 60 73.02) (end 56.5 69.52) (width 0.2) (layer "B.Cu") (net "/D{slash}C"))
 (segment (start 78.38 54.02) (end 78.38 64.64) (width 0.2) (layer "B.Cu") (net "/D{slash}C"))
 (segment (start 70 73.02) (end 60 73.02) (width 0.2) (layer "B.Cu") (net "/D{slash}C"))
 (segment (start 78.38 64.64) (end 70 73.02) (width 0.2) (layer "B.Cu") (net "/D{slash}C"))
 (segment (start 61.5 38.52) (end 62 38.52) (width 0.2) (layer "B.Cu") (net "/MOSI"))
 (segment (start 58.5 69.52) (end 58.5 41.52) (width 0.2) (layer "B.Cu") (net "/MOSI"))
 (segment (start 58.5 41.52) (end 61.5 38.52) (width 0.2) (layer "B.Cu") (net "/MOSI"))
 (segment (start 61 72.02) (end 58.5 69.52) (width 0.2) (layer "B.Cu") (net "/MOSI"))
 (segment (start 77 64.52) (end 69.5 72.02) (width 0.2) (layer "B.Cu") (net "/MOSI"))
 (segment (start 77 55.18) (end 77 64.52) (width 0.2) (layer "B.Cu") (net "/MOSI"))
 (segment (start 75.84 54.02) (end 77 55.18) (width 0.2) (layer "B.Cu") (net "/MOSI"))
 (segment (start 62.08 38.6) (end 64 38.6) (width 0.2) (layer "B.Cu") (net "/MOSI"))
 (segment (start 69.5 72.02) (end 61 72.02) (width 0.2) (layer "B.Cu") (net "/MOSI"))
 (segment (start 62 38.52) (end 62.08 38.6) (width 0.2) (layer "B.Cu") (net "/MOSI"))
 (segment (start 75 65.52) (end 69.5 71.02) (width 0.2) (layer "B.Cu") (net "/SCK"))
 (segment (start 59.5 68.42) (end 59.5 43.02) (width 0.2) (layer "B.Cu") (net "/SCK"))
 (segment (start 58.9 69.02) (end 59.5 68.42) (width 0.2) (layer "B.Cu") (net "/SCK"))
 (segment (start 75 55.72) (end 75 65.52) (width 0.2) (layer "B.Cu") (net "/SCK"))
 (segment (start 61 71.02) (end 59 69.02) (width 0.2) (layer "B.Cu") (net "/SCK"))
 (segment (start 59.5 43.02) (end 62.12 43.02) (width 0.2) (layer "B.Cu") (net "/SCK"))
 (segment (start 59 69.02) (end 58.9 69.02) (width 0.2) (layer "B.Cu") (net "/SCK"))
 (segment (start 69.5 71.02) (end 61 71.02) (width 0.2) (layer "B.Cu") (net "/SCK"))
 (segment (start 62.12 43.02) (end 64 41.14) (width 0.2) (layer "B.Cu") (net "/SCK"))
 (segment (start 73.3 54.02) (end 75 55.72) (width 0.2) (layer "B.Cu") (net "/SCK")))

